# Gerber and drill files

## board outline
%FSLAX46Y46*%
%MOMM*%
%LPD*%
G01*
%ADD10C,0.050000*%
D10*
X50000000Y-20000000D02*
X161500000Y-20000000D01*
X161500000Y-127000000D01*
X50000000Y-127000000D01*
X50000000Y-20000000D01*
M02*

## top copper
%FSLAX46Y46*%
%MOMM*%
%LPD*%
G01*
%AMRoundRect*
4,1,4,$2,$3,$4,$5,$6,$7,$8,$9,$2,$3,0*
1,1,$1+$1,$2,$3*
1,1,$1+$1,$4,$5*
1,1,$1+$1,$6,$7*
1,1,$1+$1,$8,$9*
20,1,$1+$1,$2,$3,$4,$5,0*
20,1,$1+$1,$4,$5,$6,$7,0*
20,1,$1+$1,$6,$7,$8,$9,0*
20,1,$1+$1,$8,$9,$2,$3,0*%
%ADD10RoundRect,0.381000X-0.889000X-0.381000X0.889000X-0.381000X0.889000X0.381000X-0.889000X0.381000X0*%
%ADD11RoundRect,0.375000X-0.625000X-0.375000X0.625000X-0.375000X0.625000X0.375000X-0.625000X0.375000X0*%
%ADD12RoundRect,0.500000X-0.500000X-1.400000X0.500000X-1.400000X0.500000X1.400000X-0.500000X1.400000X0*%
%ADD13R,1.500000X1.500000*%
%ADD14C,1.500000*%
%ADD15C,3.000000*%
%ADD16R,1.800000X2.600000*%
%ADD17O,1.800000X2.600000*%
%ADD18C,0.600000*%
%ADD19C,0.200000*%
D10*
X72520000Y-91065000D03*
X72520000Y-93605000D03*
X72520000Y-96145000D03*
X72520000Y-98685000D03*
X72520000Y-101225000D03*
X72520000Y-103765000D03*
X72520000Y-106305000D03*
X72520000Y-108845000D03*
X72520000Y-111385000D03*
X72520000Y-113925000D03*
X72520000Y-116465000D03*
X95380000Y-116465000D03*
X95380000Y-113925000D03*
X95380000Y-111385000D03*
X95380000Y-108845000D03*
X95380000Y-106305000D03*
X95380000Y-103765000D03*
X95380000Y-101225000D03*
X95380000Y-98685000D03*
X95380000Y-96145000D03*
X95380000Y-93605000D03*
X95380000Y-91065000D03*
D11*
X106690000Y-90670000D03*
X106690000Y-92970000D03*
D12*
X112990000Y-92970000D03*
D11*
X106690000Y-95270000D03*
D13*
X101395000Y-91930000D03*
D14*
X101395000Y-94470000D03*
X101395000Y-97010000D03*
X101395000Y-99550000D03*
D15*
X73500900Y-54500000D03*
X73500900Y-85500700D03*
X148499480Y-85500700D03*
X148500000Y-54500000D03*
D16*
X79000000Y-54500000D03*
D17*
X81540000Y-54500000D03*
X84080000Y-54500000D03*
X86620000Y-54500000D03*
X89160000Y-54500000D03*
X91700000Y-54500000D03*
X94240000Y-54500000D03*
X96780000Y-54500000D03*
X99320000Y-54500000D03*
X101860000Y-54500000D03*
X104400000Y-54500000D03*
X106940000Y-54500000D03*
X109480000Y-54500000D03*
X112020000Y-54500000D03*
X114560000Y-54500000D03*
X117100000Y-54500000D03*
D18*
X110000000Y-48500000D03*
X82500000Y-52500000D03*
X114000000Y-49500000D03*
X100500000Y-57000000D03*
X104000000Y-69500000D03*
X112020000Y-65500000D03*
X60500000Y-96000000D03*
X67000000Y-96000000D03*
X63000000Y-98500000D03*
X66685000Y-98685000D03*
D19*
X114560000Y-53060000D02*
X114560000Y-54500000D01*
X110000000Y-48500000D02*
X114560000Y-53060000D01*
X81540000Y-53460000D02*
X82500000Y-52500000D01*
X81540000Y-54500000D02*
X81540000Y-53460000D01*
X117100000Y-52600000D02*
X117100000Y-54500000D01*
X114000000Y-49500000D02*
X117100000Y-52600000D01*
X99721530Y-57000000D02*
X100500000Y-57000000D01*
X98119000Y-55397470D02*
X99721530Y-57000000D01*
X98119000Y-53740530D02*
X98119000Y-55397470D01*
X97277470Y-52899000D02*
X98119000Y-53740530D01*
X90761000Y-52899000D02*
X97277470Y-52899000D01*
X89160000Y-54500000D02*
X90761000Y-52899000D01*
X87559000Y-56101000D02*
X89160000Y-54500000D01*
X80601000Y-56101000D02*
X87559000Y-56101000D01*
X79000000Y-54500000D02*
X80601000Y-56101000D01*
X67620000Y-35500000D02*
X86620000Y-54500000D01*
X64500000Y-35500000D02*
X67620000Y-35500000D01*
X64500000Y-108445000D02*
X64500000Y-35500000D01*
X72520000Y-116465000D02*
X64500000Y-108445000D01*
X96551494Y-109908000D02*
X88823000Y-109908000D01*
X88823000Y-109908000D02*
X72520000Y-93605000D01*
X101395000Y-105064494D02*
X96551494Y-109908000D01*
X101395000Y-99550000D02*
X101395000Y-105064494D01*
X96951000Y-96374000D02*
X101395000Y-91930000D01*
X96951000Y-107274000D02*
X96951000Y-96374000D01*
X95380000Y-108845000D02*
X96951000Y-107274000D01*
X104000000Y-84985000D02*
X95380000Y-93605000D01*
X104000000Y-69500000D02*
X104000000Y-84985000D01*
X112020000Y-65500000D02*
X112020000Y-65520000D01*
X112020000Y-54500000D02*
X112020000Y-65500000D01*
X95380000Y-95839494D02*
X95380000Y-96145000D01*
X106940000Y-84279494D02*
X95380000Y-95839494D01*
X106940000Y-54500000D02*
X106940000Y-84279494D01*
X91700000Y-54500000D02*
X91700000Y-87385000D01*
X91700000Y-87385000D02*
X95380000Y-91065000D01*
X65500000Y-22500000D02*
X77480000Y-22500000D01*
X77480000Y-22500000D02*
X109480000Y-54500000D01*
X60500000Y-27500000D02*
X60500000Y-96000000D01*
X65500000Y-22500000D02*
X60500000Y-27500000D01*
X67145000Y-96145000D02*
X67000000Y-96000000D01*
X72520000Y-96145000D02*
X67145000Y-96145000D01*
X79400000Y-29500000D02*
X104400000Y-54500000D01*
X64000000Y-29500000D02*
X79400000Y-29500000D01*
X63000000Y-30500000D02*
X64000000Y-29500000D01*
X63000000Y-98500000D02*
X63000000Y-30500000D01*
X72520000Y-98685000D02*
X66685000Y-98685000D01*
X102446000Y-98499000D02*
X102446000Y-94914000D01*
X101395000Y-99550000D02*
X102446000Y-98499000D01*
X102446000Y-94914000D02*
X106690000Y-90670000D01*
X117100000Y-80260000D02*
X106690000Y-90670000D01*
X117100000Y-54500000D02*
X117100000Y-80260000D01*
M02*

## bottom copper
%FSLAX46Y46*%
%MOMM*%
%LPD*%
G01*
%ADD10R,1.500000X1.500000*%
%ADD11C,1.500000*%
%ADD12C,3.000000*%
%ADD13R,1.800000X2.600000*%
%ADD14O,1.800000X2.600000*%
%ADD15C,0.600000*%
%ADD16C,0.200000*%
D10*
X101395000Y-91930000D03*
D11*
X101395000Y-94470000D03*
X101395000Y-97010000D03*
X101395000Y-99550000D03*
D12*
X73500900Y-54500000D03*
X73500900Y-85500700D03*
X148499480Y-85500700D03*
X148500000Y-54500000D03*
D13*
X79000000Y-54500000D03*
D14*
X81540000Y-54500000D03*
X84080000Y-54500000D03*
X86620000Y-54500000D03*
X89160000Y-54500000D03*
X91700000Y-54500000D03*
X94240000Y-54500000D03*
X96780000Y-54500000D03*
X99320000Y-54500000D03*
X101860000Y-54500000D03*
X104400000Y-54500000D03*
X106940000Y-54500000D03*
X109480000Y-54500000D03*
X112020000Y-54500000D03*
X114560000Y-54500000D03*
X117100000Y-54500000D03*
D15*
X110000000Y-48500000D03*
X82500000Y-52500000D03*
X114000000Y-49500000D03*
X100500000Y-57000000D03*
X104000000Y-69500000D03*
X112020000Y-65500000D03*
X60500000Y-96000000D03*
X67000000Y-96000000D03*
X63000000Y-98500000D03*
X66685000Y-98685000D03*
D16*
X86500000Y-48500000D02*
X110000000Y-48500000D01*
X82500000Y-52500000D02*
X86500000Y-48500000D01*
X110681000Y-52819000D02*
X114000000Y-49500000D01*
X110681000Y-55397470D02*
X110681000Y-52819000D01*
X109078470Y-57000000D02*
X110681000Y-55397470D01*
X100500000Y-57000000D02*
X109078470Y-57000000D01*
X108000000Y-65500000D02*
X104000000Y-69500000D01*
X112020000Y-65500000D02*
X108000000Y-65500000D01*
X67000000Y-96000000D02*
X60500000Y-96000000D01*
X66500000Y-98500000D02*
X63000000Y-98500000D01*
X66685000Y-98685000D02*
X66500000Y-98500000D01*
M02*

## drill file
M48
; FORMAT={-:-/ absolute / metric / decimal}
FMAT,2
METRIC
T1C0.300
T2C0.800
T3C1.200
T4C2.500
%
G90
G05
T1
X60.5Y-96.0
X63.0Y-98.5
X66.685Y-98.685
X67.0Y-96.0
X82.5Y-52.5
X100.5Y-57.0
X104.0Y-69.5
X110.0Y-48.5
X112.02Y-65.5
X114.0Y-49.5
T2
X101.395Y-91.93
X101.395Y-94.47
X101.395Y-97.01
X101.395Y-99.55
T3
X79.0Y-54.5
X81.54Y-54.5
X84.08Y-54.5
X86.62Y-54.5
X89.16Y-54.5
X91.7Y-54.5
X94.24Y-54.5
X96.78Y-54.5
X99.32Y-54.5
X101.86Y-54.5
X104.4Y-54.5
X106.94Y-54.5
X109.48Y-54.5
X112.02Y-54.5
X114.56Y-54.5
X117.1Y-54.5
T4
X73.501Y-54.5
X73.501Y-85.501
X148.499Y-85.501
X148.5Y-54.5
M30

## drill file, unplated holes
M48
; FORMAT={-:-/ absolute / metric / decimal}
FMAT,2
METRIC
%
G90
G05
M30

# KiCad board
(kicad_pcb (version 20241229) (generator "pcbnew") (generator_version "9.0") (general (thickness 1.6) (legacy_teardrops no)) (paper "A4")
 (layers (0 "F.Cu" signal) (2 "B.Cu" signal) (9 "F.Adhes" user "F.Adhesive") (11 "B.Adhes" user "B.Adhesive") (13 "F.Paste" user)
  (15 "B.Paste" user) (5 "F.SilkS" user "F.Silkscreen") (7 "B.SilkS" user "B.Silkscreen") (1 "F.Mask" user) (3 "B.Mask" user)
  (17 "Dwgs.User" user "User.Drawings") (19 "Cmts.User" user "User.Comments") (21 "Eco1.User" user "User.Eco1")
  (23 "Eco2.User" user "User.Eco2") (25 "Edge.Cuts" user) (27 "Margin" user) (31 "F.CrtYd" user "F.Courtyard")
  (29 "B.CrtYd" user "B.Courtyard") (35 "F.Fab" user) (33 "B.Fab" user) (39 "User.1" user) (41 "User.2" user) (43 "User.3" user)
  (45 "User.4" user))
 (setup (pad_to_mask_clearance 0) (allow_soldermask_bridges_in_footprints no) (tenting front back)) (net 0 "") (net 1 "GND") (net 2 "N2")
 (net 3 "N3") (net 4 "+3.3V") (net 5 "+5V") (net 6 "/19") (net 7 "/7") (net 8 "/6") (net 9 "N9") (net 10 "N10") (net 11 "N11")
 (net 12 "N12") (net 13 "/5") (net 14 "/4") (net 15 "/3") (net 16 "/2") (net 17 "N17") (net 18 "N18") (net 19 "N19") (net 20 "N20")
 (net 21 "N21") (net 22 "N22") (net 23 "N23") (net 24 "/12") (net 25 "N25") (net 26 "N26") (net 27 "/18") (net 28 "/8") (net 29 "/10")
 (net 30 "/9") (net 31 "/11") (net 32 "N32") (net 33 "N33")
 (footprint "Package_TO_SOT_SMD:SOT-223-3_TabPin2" (layer "F.Cu") (at 109.84 92.97)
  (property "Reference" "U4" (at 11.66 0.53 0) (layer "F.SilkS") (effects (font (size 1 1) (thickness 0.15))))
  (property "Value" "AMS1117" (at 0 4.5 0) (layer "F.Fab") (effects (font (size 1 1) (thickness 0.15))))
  (pad "1" smd roundrect (at -3.15 -2.3) (size 2 1.5) (layers "F.Cu" "F.Mask" "F.Paste") (roundrect_rratio 0.25) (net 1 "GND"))
  (pad "2" smd roundrect (at -3.15 0) (size 2 1.5) (layers "F.Cu" "F.Mask" "F.Paste") (roundrect_rratio 0.25) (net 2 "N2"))
  (pad "2" smd roundrect (at 3.15 0) (size 2 3.8) (layers "F.Cu" "F.Mask" "F.Paste") (roundrect_rratio 0.25) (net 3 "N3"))
  (pad "3" smd roundrect (at -3.15 2.3) (size 2 1.5) (layers "F.Cu" "F.Mask" "F.Paste") (roundrect_rratio 0.25) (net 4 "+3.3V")))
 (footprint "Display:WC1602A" (layer "F.Cu") (at 79 54.5)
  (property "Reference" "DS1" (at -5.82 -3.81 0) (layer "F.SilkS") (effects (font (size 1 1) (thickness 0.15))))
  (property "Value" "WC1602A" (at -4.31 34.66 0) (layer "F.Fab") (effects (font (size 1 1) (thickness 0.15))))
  (pad "" thru_hole circle (at -5.4991 0) (size 3 3) (drill 2.5) (layers "*.Cu" "*.Mask") (remove_unused_layers no))
  (pad "" thru_hole circle (at -5.4991 31.0007) (size 3 3) (drill 2.5) (layers "*.Cu" "*.Mask") (remove_unused_layers no))
  (pad "" thru_hole circle (at 69.49948 31.0007) (size 3 3) (drill 2.5) (layers "*.Cu" "*.Mask") (remove_unused_layers no))
  (pad "" thru_hole circle (at 69.5 0) (size 3 3) (drill 2.5) (layers "*.Cu" "*.Mask") (remove_unused_layers no))
  (pad "1" thru_hole rect (at 0 0) (size 1.8 2.6) (drill 1.2) (layers "*.Cu" "*.Mask") (remove_unused_layers no) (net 1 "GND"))
  (pad "2" thru_hole oval (at 2.54 0) (size 1.8 2.6) (drill 1.2) (layers "*.Cu" "*.Mask") (remove_unused_layers no) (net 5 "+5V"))
  (pad "3" thru_hole oval (at 5.08 0) (size 1.8 2.6) (drill 1.2) (layers "*.Cu" "*.Mask") (remove_unused_layers no) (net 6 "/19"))
  (pad "4" thru_hole oval (at 7.62 0) (size 1.8 2.6) (drill 1.2) (layers "*.Cu" "*.Mask") (remove_unused_layers no) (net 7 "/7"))
  (pad "5" thru_hole oval (at 10.16 0) (size 1.8 2.6) (drill 1.2) (layers "*.Cu" "*.Mask") (remove_unused_layers no) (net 1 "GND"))
  (pad "6" thru_hole oval (at 12.7 0) (size 1.8 2.6) (drill 1.2) (layers "*.Cu" "*.Mask") (remove_unused_layers no) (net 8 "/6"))
  (pad "7" thru_hole oval (at 15.24 0) (size 1.8 2.6) (drill 1.2) (layers "*.Cu" "*.Mask") (remove_unused_layers no) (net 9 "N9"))
  (pad "8" thru_hole oval (at 17.78 0) (size 1.8 2.6) (drill 1.2) (layers "*.Cu" "*.Mask") (remove_unused_layers no) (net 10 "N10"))
  (pad "9" thru_hole oval (at 20.32 0) (size 1.8 2.6) (drill 1.2) (layers "*.Cu" "*.Mask") (remove_unused_layers no) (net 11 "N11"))
  (pad "10" thru_hole oval (at 22.86 0) (size 1.8 2.6) (drill 1.2) (layers "*.Cu" "*.Mask") (remove_unused_layers no) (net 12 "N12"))
  (pad "11" thru_hole oval (at 25.4 0) (size 1.8 2.6) (drill 1.2) (layers "*.Cu" "*.Mask") (remove_unused_layers no) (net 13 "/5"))
  (pad "12" thru_hole oval (at 27.94 0) (size 1.8 2.6) (drill 1.2) (layers "*.Cu" "*.Mask") (remove_unused_layers no) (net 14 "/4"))
  (pad "13" thru_hole oval (at 30.48 0) (size 1.8 2.6) (drill 1.2) (layers "*.Cu" "*.Mask") (remove_unused_layers no) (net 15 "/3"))
  (pad "14" thru_hole oval (at 33.02 0) (size 1.8 2.6) (drill 1.2) (layers "*.Cu" "*.Mask") (remove_unused_layers no) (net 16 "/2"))
  (pad "15" thru_hole oval (at 35.56 0) (size 1.8 2.6) (drill 1.2) (layers "*.Cu" "*.Mask") (remove_unused_layers no) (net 5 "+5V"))
  (pad "16" thru_hole oval (at 38.1 0) (size 1.8 2.6) (drill 1.2) (layers "*.Cu" "*.Mask") (remove_unused_layers no) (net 1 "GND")))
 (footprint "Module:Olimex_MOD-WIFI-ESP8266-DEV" (layer "F.Cu") (at 83.95 103.765)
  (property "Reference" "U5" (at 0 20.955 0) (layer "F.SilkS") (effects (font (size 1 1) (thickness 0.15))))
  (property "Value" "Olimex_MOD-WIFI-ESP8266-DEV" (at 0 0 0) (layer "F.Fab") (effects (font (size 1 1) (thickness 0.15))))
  (pad "1" smd roundrect (at -11.43 -12.7) (size 2.54 1.524) (layers "F.Cu" "F.Mask" "F.Paste") (roundrect_rratio 0.25) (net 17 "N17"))
  (pad "2" smd roundrect (at -11.43 -10.16) (size 2.54 1.524) (layers "F.Cu" "F.Mask" "F.Paste") (roundrect_rratio 0.25) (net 1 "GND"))
  (pad "3" smd roundrect (at -11.43 -7.62) (size 2.54 1.524) (layers "F.Cu" "F.Mask" "F.Paste") (roundrect_rratio 0.25) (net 15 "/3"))
  (pad "4" smd roundrect (at -11.43 -5.08) (size 2.54 1.524) (layers "F.Cu" "F.Mask" "F.Paste") (roundrect_rratio 0.25) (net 13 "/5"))
  (pad "5" smd roundrect (at -11.43 -2.54) (size 2.54 1.524) (layers "F.Cu" "F.Mask" "F.Paste") (roundrect_rratio 0.25) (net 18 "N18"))
  (pad "6" smd roundrect (at -11.43 0) (size 2.54 1.524) (layers "F.Cu" "F.Mask" "F.Paste") (roundrect_rratio 0.25) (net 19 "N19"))
  (pad "7" smd roundrect (at -11.43 2.54) (size 2.54 1.524) (layers "F.Cu" "F.Mask" "F.Paste") (roundrect_rratio 0.25) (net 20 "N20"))
  (pad "8" smd roundrect (at -11.43 5.08) (size 2.54 1.524) (layers "F.Cu" "F.Mask" "F.Paste") (roundrect_rratio 0.25) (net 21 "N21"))
  (pad "9" smd roundrect (at -11.43 7.62) (size 2.54 1.524) (layers "F.Cu" "F.Mask" "F.Paste") (roundrect_rratio 0.25) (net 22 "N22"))
  (pad "10" smd roundrect (at -11.43 10.16) (size 2.54 1.524) (layers "F.Cu" "F.Mask" "F.Paste") (roundrect_rratio 0.25) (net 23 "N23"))
  (pad "11" smd roundrect (at -11.43 12.7) (size 2.54 1.524) (layers "F.Cu" "F.Mask" "F.Paste") (roundrect_rratio 0.25) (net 7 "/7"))
  (pad "12" smd roundrect (at 11.43 12.7) (size 2.54 1.524) (layers "F.Cu" "F.Mask" "F.Paste") (roundrect_rratio 0.25) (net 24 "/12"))
  (pad "13" smd roundrect (at 11.43 10.16) (size 2.54 1.524) (layers "F.Cu" "F.Mask" "F.Paste") (roundrect_rratio 0.25) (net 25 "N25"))
  (pad "14" smd roundrect (at 11.43 7.62) (size 2.54 1.524) (layers "F.Cu" "F.Mask" "F.Paste") (roundrect_rratio 0.25) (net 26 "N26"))
  (pad "15" smd roundrect (at 11.43 5.08) (size 2.54 1.524) (layers "F.Cu" "F.Mask" "F.Paste") (roundrect_rratio 0.25) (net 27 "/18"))
  (pad "16" smd roundrect (at 11.43 2.54) (size 2.54 1.524) (layers "F.Cu" "F.Mask" "F.Paste") (roundrect_rratio 0.25) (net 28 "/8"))
  (pad "17" smd roundrect (at 11.43 0) (size 2.54 1.524) (layers "F.Cu" "F.Mask" "F.Paste") (roundrect_rratio 0.25) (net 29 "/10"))
  (pad "18" smd roundrect (at 11.43 -2.54) (size 2.54 1.524) (layers "F.Cu" "F.Mask" "F.Paste") (roundrect_rratio 0.25) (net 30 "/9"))
  (pad "19" smd roundrect (at 11.43 -5.08) (size 2.54 1.524) (layers "F.Cu" "F.Mask" "F.Paste") (roundrect_rratio 0.25) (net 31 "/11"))
  (pad "20" smd roundrect (at 11.43 -7.62) (size 2.54 1.524) (layers "F.Cu" "F.Mask" "F.Paste") (roundrect_rratio 0.25) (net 14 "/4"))
  (pad "21" smd roundrect (at 11.43 -10.16) (size 2.54 1.524) (layers "F.Cu" "F.Mask" "F.Paste") (roundrect_rratio 0.25) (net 16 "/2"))
  (pad "22" smd roundrect (at 11.43 -12.7) (size 2.54 1.524) (layers "F.Cu" "F.Mask" "F.Paste") (roundrect_rratio 0.25) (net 8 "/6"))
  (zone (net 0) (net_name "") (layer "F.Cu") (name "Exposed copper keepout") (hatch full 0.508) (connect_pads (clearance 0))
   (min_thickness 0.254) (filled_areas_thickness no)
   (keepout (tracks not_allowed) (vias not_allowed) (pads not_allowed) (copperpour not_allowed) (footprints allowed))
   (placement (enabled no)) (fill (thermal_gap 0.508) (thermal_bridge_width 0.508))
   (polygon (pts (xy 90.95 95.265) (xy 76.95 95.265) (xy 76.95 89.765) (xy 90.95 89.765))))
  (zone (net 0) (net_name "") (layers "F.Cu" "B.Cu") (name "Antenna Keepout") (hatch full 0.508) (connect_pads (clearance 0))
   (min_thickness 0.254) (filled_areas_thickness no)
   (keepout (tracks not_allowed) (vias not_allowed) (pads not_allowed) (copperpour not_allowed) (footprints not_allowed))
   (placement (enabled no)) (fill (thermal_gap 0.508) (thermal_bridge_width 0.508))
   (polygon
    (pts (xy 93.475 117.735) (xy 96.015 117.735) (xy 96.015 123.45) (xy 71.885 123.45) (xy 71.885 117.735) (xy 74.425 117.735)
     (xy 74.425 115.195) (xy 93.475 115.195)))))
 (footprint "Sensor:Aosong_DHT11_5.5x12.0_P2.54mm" (layer "F.Cu") (at 101.395 91.93)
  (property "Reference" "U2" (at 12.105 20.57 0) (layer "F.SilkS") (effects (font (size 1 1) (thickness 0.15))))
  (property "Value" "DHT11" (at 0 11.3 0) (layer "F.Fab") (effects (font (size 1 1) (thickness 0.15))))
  (pad "1" thru_hole rect (at 0 0) (size 1.5 1.5) (drill 0.8) (layers "*.Cu" "*.Mask") (remove_unused_layers no) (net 27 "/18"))
  (pad "2" thru_hole circle (at 0 2.54) (size 1.5 1.5) (drill 0.8) (layers "*.Cu" "*.Mask") (remove_unused_layers no) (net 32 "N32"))
  (pad "3" thru_hole circle (at 0 5.08) (size 1.5 1.5) (drill 0.8) (layers "*.Cu" "*.Mask") (remove_unused_layers no) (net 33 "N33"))
  (pad "4" thru_hole circle (at 0 7.62) (size 1.5 1.5) (drill 0.8) (layers "*.Cu" "*.Mask") (remove_unused_layers no) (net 1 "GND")))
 (gr_rect (start 50 20) (end 161.5 127) (stroke (width 0.05) (type default)) (fill no) (layer "Edge.Cuts"))
 (segment (start 117.1 54.5) (end 117.1 80.26) (width 0.2) (layer "F.Cu") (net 1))
 (segment (start 90.761 52.899) (end 97.27747 52.899) (width 0.2) (layer "F.Cu") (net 1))
 (segment (start 80.601 56.101) (end 87.559 56.101) (width 0.2) (layer "F.Cu") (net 1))
 (segment (start 97.27747 52.899) (end 98.119 53.74053) (width 0.2) (layer "F.Cu") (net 1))
 (segment (start 101.395 105.064494) (end 96.551494 109.908) (width 0.2) (layer "F.Cu") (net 1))
 (segment (start 98.119 53.74053) (end 98.119 55.39747) (width 0.2) (layer "F.Cu") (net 1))
 (segment (start 88.823 109.908) (end 72.52 93.605) (width 0.2) (layer "F.Cu") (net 1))
 (segment (start 96.551494 109.908) (end 88.823 109.908) (width 0.2) (layer "F.Cu") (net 1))
 (segment (start 101.395 99.55) (end 102.446 98.499) (width 0.2) (layer "F.Cu") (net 1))
 (segment (start 89.16 54.5) (end 90.761 52.899) (width 0.2) (layer "F.Cu") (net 1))
 (segment (start 99.72153 57) (end 100.5 57) (width 0.2) (layer "F.Cu") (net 1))
 (segment (start 98.119 55.39747) (end 99.72153 57) (width 0.2) (layer "F.Cu") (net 1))
 (segment (start 117.1 52.6) (end 117.1 54.5) (width 0.2) (layer "F.Cu") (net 1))
 (segment (start 117.1 80.26) (end 106.69 90.67) (width 0.2) (layer "F.Cu") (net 1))
 (segment (start 114 49.5) (end 117.1 52.6) (width 0.2) (layer "F.Cu") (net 1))
 (segment (start 87.559 56.101) (end 89.16 54.5) (width 0.2) (layer "F.Cu") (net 1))
 (segment (start 79 54.5) (end 80.601 56.101) (width 0.2) (layer "F.Cu") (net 1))
 (segment (start 102.446 98.499) (end 102.446 94.914) (width 0.2) (layer "F.Cu") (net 1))
 (segment (start 102.446 94.914) (end 106.69 90.67) (width 0.2) (layer "F.Cu") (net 1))
 (segment (start 101.395 99.55) (end 101.395 105.064494) (width 0.2) (layer "F.Cu") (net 1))
 (via (at 100.5 57) (size 0.6) (drill 0.3) (layers "F.Cu" "B.Cu") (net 1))
 (via (at 114 49.5) (size 0.6) (drill 0.3) (layers "F.Cu" "B.Cu") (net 1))
 (segment (start 110.681 55.39747) (end 110.681 52.819) (width 0.2) (layer "B.Cu") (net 1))
 (segment (start 110.681 52.819) (end 114 49.5) (width 0.2) (layer "B.Cu") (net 1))
 (segment (start 109.07847 57) (end 110.681 55.39747) (width 0.2) (layer "B.Cu") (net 1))
 (segment (start 100.5 57) (end 109.07847 57) (width 0.2) (layer "B.Cu") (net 1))
 (segment (start 63 98.5) (end 63 30.5) (width 0.2) (layer "F.Cu") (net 13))
 (segment (start 79.4 29.5) (end 104.4 54.5) (width 0.2) (layer "F.Cu") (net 13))
 (segment (start 64 29.5) (end 79.4 29.5) (width 0.2) (layer "F.Cu") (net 13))
 (segment (start 72.52 98.685) (end 66.685 98.685) (width 0.2) (layer "F.Cu") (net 13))
 (segment (start 63 30.5) (end 64 29.5) (width 0.2) (layer "F.Cu") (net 13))
 (via (at 63 98.5) (size 0.6) (drill 0.3) (layers "F.Cu" "B.Cu") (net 13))
 (via (at 66.685 98.685) (size 0.6) (drill 0.3) (layers "F.Cu" "B.Cu") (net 13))
 (segment (start 66.685 98.685) (end 66.5 98.5) (width 0.2) (layer "B.Cu") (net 13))
 (segment (start 66.5 98.5) (end 63 98.5) (width 0.2) (layer "B.Cu") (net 13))
 (segment (start 91.7 54.5) (end 91.7 87.385) (width 0.2) (layer "F.Cu") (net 8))
 (segment (start 91.7 87.385) (end 95.38 91.065) (width 0.2) (layer "F.Cu") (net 8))
 (segment (start 65.5 22.5) (end 60.5 27.5) (width 0.2) (layer "F.Cu") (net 15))
 (segment (start 60.5 27.5) (end 60.5 96) (width 0.2) (layer "F.Cu") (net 15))
 (segment (start 65.5 22.5) (end 77.48 22.5) (width 0.2) (layer "F.Cu") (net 15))
 (segment (start 72.52 96.145) (end 67.145 96.145) (width 0.2) (layer "F.Cu") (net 15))
 (segment (start 77.48 22.5) (end 109.48 54.5) (width 0.2) (layer "F.Cu") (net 15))
 (segment (start 67.145 96.145) (end 67 96) (width 0.2) (layer "F.Cu") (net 15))
 (via (at 60.5 96) (size 0.6) (drill 0.3) (layers "F.Cu" "B.Cu") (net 15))
 (via (at 67 96) (size 0.6) (drill 0.3) (layers "F.Cu" "B.Cu") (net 15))
 (segment (start 67 96) (end 60.5 96) (width 0.2) (layer "B.Cu") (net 15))
 (segment (start 64.5 108.445) (end 64.5 35.5) (width 0.2) (layer "F.Cu") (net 7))
 (segment (start 64.5 35.5) (end 67.62 35.5) (width 0.2) (layer "F.Cu") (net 7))
 (segment (start 67.62 35.5) (end 86.62 54.5) (width 0.2) (layer "F.Cu") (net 7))
 (segment (start 72.52 116.465) (end 64.5 108.445) (width 0.2) (layer "F.Cu") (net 7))
 (segment (start 81.54 53.46) (end 82.5 52.5) (width 0.2) (layer "F.Cu") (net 5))
 (segment (start 110 48.5) (end 114.56 53.06) (width 0.2) (layer "F.Cu") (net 5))
 (segment (start 81.54 54.5) (end 81.54 53.46) (width 0.2) (layer "F.Cu") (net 5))
 (segment (start 114.56 53.06) (end 114.56 54.5) (width 0.2) (layer "F.Cu") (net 5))
 (via (at 82.5 52.5) (size 0.6) (drill 0.3) (layers "F.Cu" "B.Cu") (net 5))
 (via (at 110 48.5) (size 0.6) (drill 0.3) (layers "F.Cu" "B.Cu") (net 5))
 (segment (start 82.5 52.5) (end 86.5 48.5) (width 0.2) (layer "B.Cu") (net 5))
 (segment (start 86.5 48.5) (end 110 48.5) (width 0.2) (layer "B.Cu") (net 5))
 (segment (start 112.02 54.5) (end 112.02 65.5) (width 0.2) (layer "F.Cu") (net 16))
 (segment (start 104 84.985) (end 95.38 93.605) (width 0.2) (layer "F.Cu") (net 16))
 (segment (start 104 69.5) (end 104 84.985) (width 0.2) (layer "F.Cu") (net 16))
 (segment (start 112.02 65.5) (end 112.02 65.52) (width 0.2) (layer "F.Cu") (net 16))
 (via (at 104 69.5) (size 0.6) (drill 0.3) (layers "F.Cu" "B.Cu") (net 16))
 (via (at 112.02 65.5) (size 0.6) (drill 0.3) (layers "F.Cu" "B.Cu") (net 16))
 (segment (start 108 65.5) (end 104 69.5) (width 0.2) (layer "B.Cu") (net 16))
 (segment (start 112.02 65.5) (end 108 65.5) (width 0.2) (layer "B.Cu") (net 16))
 (segment (start 106.94 84.279494) (end 95.38 95.839494) (width 0.2) (layer "F.Cu") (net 14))
 (segment (start 95.38 95.839494) (end 95.38 96.145) (width 0.2) (layer "F.Cu") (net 14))
 (segment (start 106.94 54.5) (end 106.94 84.279494) (width 0.2) (layer "F.Cu") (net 14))
 (segment (start 95.38 108.845) (end 96.951 107.274) (width 0.2) (layer "F.Cu") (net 27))
 (segment (start 96.951 96.374) (end 101.395 91.93) (width 0.2) (layer "F.Cu") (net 27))
 (segment (start 96.951 107.274) (end 96.951 96.374) (width 0.2) (layer "F.Cu") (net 27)))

